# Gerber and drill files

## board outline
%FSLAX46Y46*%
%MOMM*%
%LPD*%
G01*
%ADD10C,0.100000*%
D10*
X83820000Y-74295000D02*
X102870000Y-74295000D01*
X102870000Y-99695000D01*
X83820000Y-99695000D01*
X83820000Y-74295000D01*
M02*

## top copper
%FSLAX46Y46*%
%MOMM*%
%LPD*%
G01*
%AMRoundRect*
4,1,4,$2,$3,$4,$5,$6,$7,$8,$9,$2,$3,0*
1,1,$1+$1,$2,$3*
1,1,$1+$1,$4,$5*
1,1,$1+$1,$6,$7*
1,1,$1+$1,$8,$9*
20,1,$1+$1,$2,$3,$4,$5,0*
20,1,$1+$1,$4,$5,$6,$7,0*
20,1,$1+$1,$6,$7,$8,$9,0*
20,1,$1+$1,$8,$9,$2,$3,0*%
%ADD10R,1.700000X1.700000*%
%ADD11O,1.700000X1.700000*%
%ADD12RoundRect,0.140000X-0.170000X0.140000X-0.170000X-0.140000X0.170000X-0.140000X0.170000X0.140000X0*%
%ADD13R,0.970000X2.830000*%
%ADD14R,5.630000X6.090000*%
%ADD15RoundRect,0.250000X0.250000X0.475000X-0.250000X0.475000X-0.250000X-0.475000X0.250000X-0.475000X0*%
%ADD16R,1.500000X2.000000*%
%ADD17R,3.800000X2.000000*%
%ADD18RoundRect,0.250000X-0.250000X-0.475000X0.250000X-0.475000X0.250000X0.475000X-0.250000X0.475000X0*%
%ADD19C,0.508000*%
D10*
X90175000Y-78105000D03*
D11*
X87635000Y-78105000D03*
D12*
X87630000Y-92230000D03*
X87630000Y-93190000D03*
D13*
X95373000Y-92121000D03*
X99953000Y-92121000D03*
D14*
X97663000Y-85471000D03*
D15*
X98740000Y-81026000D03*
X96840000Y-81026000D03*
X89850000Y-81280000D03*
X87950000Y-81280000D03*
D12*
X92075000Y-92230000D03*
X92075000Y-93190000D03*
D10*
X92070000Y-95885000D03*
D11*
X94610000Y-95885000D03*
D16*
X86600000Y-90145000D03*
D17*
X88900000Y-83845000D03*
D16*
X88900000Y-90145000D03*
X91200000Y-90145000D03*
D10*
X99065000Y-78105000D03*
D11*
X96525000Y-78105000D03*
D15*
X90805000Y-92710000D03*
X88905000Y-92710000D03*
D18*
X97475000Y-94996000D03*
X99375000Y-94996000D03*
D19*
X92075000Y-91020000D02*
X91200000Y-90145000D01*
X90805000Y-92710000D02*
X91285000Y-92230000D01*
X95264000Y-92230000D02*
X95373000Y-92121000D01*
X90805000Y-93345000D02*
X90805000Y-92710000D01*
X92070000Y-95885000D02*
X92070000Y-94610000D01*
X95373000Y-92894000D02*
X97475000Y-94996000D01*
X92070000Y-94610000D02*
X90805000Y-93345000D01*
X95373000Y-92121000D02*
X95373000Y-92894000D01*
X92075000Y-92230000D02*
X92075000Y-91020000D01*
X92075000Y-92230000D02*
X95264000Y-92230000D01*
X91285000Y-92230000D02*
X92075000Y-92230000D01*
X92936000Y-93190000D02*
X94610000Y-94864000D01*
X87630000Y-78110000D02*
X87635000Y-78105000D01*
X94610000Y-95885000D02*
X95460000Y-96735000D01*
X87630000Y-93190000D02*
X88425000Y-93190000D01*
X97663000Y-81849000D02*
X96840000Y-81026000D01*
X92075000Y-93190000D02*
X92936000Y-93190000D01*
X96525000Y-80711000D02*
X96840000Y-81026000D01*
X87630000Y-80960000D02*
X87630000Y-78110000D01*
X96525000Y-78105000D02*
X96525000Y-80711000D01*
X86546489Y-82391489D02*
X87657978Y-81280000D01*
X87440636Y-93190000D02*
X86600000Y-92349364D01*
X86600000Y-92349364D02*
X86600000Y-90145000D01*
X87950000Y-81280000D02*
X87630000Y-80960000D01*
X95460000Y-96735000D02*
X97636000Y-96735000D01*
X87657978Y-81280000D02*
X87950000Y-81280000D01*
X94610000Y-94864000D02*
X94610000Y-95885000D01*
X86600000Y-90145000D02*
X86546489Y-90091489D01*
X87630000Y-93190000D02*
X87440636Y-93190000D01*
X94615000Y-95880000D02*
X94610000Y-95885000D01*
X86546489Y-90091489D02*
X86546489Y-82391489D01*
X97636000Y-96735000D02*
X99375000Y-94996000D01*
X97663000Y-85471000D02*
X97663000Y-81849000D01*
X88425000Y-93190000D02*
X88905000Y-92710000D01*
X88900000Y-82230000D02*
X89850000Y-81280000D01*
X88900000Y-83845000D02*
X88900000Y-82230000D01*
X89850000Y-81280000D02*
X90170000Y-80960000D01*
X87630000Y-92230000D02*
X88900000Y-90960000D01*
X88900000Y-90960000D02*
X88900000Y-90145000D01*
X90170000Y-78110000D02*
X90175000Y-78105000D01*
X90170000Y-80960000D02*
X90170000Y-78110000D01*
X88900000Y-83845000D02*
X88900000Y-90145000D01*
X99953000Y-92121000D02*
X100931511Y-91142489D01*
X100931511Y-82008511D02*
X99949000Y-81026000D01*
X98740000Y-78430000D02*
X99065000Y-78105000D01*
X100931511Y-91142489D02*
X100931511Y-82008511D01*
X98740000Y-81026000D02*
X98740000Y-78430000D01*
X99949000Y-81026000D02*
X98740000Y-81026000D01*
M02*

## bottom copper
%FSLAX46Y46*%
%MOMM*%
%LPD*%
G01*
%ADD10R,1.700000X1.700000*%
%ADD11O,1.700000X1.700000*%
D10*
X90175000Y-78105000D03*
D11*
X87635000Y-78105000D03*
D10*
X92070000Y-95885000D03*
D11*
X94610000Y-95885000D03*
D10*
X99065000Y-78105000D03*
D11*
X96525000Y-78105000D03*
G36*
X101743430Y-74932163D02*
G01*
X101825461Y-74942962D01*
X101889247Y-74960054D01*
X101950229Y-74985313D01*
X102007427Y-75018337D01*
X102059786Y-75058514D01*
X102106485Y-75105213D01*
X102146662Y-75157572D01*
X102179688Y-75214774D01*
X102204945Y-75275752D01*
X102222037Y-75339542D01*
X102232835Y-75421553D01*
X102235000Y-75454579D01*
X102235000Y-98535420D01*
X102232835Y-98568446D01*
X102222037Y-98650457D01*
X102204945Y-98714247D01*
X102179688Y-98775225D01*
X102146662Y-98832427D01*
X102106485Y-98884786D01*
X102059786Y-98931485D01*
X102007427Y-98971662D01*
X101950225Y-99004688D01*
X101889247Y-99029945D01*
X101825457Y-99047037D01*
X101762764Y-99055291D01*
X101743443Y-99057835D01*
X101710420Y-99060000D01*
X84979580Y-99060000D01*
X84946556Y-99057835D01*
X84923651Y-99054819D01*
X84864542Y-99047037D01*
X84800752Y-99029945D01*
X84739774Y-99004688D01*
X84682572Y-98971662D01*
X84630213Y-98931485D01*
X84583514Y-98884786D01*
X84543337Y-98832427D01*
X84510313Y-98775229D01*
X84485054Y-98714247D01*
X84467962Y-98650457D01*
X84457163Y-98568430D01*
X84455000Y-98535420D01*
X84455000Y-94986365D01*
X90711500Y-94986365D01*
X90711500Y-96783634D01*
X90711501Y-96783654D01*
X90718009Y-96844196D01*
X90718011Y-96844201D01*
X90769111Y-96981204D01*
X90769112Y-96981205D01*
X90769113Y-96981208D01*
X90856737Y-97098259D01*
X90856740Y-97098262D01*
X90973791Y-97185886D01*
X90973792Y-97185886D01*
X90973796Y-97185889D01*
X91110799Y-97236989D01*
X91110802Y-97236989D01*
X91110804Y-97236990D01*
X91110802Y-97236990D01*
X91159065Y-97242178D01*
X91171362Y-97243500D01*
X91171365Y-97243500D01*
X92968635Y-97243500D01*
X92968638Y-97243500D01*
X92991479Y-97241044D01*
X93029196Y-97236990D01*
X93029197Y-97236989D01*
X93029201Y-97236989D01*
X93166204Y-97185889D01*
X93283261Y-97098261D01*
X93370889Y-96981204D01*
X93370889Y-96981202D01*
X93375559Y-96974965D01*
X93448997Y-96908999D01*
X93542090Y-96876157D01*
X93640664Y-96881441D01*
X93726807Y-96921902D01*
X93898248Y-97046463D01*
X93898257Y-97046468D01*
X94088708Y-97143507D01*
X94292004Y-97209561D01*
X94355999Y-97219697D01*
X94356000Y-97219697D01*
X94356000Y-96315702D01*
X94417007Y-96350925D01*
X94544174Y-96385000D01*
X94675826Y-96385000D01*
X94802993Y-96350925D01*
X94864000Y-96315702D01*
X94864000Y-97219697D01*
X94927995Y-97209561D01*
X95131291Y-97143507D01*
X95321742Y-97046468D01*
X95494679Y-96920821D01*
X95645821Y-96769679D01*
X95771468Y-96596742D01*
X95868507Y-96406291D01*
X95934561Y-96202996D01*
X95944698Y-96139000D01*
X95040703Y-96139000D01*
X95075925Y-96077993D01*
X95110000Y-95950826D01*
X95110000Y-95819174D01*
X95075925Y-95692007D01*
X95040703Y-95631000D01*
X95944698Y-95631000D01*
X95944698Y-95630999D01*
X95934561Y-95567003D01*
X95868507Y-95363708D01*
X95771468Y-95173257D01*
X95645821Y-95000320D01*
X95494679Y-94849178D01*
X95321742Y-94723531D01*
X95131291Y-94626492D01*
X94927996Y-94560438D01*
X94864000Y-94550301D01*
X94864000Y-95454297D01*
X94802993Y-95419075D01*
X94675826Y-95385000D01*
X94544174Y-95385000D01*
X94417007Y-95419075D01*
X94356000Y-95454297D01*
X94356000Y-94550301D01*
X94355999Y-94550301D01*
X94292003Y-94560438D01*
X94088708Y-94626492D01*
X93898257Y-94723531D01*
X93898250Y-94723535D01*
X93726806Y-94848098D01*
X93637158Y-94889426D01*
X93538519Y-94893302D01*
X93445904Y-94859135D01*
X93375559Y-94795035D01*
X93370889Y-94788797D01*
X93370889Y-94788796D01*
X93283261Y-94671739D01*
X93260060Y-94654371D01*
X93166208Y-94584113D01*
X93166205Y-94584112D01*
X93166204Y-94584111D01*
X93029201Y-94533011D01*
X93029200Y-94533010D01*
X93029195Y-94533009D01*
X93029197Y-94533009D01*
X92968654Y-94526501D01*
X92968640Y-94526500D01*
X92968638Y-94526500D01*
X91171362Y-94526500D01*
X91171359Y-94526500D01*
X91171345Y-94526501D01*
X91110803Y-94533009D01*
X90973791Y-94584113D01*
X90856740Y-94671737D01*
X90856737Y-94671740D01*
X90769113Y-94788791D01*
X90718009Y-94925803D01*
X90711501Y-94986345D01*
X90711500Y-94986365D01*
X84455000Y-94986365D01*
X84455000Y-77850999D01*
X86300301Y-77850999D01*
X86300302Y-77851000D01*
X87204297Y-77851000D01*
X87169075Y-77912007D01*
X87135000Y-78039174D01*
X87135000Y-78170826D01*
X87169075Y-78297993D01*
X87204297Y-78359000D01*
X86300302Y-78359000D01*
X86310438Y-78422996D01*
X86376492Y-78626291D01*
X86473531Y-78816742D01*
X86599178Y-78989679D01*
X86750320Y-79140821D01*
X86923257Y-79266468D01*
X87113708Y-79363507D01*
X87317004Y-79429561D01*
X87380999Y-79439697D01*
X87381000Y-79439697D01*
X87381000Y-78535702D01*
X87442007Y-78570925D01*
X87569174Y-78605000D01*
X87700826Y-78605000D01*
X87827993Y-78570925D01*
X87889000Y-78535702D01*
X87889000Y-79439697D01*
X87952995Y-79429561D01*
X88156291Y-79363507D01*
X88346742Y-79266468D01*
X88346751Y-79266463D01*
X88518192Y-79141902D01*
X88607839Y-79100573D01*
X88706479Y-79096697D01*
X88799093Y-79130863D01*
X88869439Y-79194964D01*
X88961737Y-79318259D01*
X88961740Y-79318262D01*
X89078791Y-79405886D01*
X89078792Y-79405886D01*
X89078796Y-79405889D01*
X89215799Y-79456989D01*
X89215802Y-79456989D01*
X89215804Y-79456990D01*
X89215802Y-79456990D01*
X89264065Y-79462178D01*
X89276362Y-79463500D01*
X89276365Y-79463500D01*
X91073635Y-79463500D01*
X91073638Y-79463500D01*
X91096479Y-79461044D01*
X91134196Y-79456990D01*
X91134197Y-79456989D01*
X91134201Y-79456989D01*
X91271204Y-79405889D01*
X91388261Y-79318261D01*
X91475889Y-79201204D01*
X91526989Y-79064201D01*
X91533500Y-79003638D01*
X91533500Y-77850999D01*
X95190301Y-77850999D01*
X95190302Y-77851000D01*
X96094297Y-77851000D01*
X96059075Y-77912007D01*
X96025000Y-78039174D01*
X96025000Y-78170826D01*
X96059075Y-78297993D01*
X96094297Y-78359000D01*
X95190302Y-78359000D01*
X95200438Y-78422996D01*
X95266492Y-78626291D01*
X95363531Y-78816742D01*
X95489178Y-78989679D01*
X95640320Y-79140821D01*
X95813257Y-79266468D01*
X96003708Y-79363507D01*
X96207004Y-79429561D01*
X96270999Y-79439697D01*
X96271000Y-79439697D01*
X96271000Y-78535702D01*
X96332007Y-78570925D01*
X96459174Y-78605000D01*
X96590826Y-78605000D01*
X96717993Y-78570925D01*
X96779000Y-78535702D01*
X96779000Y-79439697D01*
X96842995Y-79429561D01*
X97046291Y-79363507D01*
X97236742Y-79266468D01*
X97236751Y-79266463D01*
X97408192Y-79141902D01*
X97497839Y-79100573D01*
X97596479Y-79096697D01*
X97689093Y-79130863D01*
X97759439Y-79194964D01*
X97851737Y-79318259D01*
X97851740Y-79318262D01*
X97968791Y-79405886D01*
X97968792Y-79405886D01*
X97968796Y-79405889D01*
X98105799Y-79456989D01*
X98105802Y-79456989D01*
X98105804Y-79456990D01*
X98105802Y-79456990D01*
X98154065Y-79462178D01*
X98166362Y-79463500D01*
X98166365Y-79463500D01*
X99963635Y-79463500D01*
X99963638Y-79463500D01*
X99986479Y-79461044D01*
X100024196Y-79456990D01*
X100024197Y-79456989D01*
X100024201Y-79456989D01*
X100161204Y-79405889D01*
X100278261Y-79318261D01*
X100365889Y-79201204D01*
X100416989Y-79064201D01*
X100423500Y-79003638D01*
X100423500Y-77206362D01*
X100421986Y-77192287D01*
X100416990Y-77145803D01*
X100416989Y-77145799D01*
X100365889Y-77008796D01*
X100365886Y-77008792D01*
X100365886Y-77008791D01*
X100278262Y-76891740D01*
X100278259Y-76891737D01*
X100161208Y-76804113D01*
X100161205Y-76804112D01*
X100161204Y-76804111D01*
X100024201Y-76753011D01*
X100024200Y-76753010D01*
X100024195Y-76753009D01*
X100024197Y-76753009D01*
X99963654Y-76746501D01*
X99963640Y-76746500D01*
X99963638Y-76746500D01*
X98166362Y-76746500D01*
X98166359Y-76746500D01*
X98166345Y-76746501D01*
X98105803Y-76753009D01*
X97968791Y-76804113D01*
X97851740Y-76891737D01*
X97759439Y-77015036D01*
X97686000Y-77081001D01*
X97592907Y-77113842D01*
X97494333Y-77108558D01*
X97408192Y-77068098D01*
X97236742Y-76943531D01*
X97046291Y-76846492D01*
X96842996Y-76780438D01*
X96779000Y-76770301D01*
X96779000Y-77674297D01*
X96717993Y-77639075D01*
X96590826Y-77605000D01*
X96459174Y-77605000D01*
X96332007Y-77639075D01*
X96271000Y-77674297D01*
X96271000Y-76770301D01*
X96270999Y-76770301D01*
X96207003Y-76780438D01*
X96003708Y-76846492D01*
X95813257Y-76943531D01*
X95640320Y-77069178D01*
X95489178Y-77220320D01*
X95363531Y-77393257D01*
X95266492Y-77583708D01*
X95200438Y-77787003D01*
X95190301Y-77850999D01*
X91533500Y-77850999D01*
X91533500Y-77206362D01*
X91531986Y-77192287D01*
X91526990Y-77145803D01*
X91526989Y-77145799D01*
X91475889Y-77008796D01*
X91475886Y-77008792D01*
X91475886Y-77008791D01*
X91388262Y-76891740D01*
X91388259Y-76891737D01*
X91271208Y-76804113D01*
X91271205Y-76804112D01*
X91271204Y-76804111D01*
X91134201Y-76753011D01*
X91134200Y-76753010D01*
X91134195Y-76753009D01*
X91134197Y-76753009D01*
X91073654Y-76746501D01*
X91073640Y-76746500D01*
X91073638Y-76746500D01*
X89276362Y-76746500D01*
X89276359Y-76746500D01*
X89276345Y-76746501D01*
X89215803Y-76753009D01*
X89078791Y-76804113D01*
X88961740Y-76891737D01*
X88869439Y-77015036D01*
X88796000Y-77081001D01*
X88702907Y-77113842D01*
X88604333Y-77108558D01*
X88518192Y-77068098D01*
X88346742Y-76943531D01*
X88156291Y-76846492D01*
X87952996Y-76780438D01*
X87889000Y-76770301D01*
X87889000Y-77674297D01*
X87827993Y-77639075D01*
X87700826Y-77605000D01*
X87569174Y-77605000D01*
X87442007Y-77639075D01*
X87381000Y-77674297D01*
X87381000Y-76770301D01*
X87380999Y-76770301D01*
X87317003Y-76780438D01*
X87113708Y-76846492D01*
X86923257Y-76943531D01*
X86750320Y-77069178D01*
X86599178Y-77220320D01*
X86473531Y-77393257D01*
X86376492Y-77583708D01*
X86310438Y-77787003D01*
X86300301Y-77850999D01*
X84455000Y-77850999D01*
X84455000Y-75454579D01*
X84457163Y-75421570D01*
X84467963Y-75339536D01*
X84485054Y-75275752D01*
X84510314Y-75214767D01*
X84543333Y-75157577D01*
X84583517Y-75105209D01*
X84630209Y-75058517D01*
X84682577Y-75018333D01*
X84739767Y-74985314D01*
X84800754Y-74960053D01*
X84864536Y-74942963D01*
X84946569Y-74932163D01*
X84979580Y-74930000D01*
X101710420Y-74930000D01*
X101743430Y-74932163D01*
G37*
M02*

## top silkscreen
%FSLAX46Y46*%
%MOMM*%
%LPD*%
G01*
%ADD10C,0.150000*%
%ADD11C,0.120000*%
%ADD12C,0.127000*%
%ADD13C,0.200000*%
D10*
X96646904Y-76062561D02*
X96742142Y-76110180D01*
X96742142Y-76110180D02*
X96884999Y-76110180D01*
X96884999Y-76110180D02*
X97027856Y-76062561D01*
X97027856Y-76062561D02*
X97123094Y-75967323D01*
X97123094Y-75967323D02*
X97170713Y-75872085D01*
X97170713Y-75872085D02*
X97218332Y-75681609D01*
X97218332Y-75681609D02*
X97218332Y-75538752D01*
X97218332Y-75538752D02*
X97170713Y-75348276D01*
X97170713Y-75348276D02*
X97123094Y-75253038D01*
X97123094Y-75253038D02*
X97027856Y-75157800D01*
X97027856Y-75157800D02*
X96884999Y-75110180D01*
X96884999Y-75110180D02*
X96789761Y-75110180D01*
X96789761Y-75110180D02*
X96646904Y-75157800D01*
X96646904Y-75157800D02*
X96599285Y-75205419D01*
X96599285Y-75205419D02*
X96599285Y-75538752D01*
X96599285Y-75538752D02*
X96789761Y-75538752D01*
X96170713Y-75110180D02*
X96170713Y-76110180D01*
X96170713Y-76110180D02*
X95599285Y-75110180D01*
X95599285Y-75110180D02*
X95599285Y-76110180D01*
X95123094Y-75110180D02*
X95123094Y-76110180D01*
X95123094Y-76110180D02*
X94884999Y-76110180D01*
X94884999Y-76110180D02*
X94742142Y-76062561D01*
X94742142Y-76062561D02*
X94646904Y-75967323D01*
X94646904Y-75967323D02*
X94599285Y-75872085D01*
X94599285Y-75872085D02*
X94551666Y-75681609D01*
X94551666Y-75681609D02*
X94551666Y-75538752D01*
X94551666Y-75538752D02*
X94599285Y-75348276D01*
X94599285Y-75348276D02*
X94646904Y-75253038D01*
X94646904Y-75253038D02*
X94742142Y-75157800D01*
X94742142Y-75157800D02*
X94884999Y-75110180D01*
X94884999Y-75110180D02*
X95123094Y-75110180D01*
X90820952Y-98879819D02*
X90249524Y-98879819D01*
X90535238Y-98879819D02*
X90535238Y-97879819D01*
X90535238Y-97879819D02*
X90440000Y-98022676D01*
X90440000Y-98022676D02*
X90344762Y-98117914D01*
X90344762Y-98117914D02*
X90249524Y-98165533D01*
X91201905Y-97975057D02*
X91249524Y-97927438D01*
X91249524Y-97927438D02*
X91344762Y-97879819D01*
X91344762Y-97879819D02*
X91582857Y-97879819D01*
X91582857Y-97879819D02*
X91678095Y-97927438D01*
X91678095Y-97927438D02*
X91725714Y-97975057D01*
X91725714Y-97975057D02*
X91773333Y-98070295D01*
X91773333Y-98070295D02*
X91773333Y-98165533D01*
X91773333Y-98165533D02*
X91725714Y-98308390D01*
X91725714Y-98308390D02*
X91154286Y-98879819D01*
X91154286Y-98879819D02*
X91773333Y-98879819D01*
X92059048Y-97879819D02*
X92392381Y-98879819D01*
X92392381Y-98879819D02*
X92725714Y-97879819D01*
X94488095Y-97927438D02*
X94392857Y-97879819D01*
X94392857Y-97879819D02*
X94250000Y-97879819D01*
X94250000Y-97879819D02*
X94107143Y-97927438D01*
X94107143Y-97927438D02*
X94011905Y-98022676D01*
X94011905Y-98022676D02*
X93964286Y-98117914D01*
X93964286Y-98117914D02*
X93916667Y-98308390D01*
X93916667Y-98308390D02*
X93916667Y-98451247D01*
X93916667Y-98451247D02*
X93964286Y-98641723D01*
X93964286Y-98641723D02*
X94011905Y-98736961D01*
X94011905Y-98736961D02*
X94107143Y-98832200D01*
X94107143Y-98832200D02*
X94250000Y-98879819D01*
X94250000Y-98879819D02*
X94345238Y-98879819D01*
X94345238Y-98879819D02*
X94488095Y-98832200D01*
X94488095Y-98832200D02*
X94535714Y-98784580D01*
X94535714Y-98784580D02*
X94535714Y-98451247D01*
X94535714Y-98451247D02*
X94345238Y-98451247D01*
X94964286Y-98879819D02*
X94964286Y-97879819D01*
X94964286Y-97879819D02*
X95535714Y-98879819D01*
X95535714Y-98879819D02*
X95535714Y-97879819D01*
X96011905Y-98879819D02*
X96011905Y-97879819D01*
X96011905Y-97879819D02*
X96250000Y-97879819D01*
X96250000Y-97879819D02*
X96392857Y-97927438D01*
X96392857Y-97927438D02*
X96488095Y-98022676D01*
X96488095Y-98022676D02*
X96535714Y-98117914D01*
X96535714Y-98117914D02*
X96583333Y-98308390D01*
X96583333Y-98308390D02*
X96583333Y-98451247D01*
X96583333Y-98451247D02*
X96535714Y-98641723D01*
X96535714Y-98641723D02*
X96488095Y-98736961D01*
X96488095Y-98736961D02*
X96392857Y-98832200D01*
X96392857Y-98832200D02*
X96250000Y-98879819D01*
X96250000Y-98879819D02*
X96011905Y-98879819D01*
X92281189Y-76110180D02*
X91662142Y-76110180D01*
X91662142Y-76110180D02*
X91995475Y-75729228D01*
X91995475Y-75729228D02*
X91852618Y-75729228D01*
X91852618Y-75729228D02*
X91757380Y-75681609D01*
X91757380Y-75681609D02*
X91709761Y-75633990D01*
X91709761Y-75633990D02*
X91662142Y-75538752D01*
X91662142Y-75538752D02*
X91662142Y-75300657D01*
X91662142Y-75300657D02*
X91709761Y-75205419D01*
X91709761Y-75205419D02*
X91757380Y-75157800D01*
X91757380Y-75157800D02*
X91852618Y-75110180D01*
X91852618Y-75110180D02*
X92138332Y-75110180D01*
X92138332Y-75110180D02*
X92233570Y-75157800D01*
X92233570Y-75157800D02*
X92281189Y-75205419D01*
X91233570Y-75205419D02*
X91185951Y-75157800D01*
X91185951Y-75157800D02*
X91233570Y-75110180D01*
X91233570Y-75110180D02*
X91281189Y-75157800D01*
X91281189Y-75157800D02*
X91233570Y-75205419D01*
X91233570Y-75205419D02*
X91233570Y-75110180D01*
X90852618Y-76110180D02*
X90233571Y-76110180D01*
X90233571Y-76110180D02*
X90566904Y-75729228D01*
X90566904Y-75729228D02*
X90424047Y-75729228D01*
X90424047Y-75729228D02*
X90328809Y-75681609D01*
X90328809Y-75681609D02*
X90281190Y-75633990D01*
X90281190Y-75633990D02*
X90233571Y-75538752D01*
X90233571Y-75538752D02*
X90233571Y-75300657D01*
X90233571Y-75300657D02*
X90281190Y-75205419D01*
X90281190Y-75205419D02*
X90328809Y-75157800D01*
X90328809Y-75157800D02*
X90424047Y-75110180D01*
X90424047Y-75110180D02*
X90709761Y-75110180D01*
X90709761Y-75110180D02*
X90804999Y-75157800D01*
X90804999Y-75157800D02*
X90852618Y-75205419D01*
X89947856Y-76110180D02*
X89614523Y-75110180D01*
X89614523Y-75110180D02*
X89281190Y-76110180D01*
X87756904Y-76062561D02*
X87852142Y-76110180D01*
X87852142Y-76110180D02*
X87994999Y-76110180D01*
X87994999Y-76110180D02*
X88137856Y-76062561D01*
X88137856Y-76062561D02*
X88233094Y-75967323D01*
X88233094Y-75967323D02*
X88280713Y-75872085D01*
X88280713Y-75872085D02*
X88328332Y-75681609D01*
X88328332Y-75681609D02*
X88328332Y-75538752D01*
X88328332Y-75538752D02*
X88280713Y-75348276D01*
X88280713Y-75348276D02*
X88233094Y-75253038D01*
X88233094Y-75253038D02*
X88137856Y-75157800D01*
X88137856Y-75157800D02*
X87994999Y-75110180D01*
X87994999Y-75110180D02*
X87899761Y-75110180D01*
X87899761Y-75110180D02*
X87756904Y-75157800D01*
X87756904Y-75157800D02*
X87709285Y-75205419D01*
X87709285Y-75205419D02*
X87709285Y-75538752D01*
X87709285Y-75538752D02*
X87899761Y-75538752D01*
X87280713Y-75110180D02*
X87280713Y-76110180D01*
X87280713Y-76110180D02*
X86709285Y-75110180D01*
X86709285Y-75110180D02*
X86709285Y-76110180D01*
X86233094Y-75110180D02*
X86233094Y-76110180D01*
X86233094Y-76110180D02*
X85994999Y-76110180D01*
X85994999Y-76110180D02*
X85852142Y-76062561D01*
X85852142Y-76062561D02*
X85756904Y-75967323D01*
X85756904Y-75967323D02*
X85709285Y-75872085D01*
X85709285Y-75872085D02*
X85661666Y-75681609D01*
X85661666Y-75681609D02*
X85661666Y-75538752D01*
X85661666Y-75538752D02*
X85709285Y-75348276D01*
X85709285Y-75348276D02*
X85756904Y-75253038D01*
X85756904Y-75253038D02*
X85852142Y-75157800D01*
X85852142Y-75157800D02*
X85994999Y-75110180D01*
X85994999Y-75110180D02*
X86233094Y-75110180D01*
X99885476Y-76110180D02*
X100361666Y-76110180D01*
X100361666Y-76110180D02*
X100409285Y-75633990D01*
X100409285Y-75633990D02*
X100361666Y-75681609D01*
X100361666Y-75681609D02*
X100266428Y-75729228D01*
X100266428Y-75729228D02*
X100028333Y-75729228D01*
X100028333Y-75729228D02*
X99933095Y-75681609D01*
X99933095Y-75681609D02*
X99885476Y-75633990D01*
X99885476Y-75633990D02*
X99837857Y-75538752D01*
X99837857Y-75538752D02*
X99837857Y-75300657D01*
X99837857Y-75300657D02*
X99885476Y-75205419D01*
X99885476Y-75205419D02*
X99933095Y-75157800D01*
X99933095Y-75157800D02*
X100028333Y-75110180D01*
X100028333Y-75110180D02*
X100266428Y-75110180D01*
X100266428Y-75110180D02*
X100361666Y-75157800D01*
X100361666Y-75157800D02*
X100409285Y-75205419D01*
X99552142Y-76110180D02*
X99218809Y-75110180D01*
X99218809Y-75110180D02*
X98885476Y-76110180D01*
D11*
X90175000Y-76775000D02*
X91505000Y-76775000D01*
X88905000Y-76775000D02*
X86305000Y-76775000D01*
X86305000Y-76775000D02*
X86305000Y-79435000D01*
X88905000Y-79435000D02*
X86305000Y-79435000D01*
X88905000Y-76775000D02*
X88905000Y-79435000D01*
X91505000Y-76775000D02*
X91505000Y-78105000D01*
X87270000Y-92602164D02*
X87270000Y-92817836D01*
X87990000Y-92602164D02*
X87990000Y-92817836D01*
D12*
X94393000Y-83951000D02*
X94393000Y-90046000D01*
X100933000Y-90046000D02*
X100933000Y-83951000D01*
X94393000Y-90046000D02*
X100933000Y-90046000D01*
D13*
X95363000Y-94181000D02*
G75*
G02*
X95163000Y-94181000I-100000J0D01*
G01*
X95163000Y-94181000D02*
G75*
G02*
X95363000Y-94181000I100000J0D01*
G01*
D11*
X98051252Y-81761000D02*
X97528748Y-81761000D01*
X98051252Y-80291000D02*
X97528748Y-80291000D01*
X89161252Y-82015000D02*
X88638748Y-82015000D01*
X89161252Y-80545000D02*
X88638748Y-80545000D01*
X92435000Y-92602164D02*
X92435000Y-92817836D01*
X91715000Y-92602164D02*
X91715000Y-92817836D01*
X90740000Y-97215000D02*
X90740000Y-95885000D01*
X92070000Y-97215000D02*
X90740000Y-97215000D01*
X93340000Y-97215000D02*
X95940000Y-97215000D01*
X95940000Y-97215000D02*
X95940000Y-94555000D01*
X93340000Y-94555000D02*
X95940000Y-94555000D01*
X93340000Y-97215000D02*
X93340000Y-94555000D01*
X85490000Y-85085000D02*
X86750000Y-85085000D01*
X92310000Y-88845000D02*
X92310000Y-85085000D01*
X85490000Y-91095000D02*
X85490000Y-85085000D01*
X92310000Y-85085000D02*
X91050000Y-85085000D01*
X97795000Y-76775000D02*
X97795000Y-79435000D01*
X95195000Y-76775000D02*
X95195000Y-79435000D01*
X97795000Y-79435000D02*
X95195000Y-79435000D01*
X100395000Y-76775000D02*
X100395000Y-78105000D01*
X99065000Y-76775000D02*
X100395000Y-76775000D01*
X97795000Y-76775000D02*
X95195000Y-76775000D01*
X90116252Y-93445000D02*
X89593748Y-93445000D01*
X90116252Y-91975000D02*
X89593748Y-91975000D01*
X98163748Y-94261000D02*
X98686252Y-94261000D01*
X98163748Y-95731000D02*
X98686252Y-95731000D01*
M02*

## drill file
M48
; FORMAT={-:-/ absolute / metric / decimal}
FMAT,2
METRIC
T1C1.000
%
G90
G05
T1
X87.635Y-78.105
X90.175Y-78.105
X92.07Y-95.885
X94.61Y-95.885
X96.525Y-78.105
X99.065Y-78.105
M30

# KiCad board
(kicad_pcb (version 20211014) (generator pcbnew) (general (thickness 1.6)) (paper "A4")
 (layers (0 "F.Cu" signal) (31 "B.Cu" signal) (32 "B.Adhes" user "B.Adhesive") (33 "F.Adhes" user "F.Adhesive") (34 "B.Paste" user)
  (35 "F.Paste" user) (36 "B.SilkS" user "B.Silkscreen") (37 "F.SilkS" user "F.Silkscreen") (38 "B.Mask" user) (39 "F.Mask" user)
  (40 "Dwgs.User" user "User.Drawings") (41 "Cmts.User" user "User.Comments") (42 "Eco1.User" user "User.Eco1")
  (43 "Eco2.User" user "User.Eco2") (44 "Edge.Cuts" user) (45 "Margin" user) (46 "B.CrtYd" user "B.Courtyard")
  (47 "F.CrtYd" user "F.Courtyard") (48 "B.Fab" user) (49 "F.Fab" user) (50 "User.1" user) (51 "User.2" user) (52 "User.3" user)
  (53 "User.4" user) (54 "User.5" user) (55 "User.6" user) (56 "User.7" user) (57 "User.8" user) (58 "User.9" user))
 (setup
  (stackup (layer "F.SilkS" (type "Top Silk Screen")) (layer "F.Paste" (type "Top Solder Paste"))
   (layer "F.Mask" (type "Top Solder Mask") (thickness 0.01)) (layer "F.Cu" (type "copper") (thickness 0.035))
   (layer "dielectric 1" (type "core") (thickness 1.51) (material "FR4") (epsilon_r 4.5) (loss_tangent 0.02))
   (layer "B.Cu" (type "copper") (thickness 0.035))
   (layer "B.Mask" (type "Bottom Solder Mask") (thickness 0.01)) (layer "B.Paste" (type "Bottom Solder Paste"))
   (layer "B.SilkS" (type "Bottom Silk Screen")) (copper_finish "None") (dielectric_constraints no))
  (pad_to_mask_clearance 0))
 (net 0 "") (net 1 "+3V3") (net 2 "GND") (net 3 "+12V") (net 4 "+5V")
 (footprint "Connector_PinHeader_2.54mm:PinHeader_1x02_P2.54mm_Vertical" (layer "F.Cu") (at 90.175 78.105 -90)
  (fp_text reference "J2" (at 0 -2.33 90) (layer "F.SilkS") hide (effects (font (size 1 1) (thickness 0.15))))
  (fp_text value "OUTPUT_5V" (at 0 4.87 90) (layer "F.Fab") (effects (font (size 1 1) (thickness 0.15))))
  (fp_line (start -1.33 0) (end -1.33 -1.33) (layer "F.SilkS") (width 0.12))
  (fp_line (start -1.33 1.27) (end -1.33 3.87) (layer "F.SilkS") (width 0.12))
  (fp_line (start -1.33 3.87) (end 1.33 3.87) (layer "F.SilkS") (width 0.12))
  (fp_line (start 1.33 1.27) (end 1.33 3.87) (layer "F.SilkS") (width 0.12))
  (fp_line (start -1.33 1.27) (end 1.33 1.27) (layer "F.SilkS") (width 0.12))
  (fp_line (start -1.33 -1.33) (end 0 -1.33) (layer "F.SilkS") (width 0.12))
  (pad "1" thru_hole rect (at 0 0 270) (size 1.7 1.7) (drill 1) (layers *.Cu *.Mask) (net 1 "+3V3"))
  (pad "2" thru_hole oval (at 0 2.54 270) (size 1.7 1.7) (drill 1) (layers *.Cu *.Mask) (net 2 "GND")))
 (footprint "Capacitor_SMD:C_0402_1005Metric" (layer "F.Cu") (at 87.63 92.71 -90)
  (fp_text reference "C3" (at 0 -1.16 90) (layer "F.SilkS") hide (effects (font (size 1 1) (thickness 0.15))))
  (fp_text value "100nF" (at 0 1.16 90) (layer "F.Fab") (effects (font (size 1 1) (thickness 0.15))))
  (fp_line (start -0.107836 0.36) (end 0.107836 0.36) (layer "F.SilkS") (width 0.12))
  (fp_line (start -0.107836 -0.36) (end 0.107836 -0.36) (layer "F.SilkS") (width 0.12))
  (pad "1" smd roundrect (at -0.48 0 270) (size 0.56 0.62) (layers "F.Cu" "F.Paste" "F.Mask") (roundrect_rratio 0.25) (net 1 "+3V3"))
  (pad "2" smd roundrect (at 0.48 0 270) (size 0.56 0.62) (layers "F.Cu" "F.Paste" "F.Mask") (roundrect_rratio 0.25) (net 2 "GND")))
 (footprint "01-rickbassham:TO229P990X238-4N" (layer "F.Cu") (at 97.663 87.981 90)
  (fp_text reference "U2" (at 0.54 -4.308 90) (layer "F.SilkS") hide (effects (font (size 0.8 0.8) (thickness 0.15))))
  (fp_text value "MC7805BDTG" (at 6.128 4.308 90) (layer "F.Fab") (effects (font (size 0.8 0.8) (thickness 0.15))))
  (fp_line (start 4.03 -3.27) (end -2.065 -3.27) (layer "F.SilkS") (width 0.127))
  (fp_line (start -2.065 3.27) (end 4.03 3.27) (layer "F.SilkS") (width 0.127))
  (fp_line (start -2.065 -3.27) (end -2.065 3.27) (layer "F.SilkS") (width 0.127))
  (fp_circle (center -6.2 -2.4) (end -6.1 -2.4) (layer "F.SilkS") (width 0.2) (fill none))
  (pad "1" smd rect (at -4.14 -2.29 90) (size 2.83 0.97) (layers "F.Cu" "F.Paste" "F.Mask") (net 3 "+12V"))
  (pad "3" smd rect (at -4.14 2.29 90) (size 2.83 0.97) (layers "F.Cu" "F.Paste" "F.Mask") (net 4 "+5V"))
  (pad "4" smd rect (at 2.51 0 90) (size 6.09 5.63) (layers "F.Cu" "F.Mask") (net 2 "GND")))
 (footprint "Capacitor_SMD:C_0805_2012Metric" (layer "F.Cu") (at 97.79 81.026 180)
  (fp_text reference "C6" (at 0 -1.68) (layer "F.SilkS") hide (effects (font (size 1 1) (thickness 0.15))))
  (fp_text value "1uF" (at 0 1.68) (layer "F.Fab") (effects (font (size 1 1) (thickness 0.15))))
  (fp_line (start -0.261252 -0.735) (end 0.261252 -0.735) (layer "F.SilkS") (width 0.12))
  (fp_line (start -0.261252 0.735) (end 0.261252 0.735) (layer "F.SilkS") (width 0.12))
  (pad "1" smd roundrect (at -0.95 0 180) (size 1 1.45) (layers "F.Cu" "F.Paste" "F.Mask") (roundrect_rratio 0.25) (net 4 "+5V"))
  (pad "2" smd roundrect (at 0.95 0 180) (size 1 1.45) (layers "F.Cu" "F.Paste" "F.Mask") (roundrect_rratio 0.25) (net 2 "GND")))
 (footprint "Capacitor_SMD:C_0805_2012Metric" (layer "F.Cu") (at 88.9 81.28 180)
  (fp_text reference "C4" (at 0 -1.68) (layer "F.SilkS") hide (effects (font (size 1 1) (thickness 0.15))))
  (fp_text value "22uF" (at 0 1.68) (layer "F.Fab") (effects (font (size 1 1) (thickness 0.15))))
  (fp_line (start -0.261252 -0.735) (end 0.261252 -0.735) (layer "F.SilkS") (width 0.12))
  (fp_line (start -0.261252 0.735) (end 0.261252 0.735) (layer "F.SilkS") (width 0.12))
  (pad "1" smd roundrect (at -0.95 0 180) (size 1 1.45) (layers "F.Cu" "F.Paste" "F.Mask") (roundrect_rratio 0.25) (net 1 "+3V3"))
  (pad "2" smd roundrect (at 0.95 0 180) (size 1 1.45) (layers "F.Cu" "F.Paste" "F.Mask") (roundrect_rratio 0.25) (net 2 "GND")))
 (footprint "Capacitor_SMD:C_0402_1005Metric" (layer "F.Cu") (at 92.075 92.71 -90)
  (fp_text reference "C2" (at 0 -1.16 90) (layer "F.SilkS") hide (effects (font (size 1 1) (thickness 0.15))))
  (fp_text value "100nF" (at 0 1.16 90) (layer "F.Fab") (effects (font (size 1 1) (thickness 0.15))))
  (fp_line (start -0.107836 -0.36) (end 0.107836 -0.36) (layer "F.SilkS") (width 0.12))
  (fp_line (start -0.107836 0.36) (end 0.107836 0.36) (layer "F.SilkS") (width 0.12))
  (pad "1" smd roundrect (at -0.48 0 270) (size 0.56 0.62) (layers "F.Cu" "F.Paste" "F.Mask") (roundrect_rratio 0.25) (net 3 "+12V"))
  (pad "2" smd roundrect (at 0.48 0 270) (size 0.56 0.62) (layers "F.Cu" "F.Paste" "F.Mask") (roundrect_rratio 0.25) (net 2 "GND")))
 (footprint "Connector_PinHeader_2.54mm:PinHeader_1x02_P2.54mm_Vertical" (layer "F.Cu") (at 92.07 95.885 90)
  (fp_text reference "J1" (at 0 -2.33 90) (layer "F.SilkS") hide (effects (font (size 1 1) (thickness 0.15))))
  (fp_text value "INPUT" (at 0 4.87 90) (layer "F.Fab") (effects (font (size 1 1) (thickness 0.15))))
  (fp_line (start -1.33 -1.33) (end 0 -1.33) (layer "F.SilkS") (width 0.12))
  (fp_line (start -1.33 0) (end -1.33 -1.33) (layer "F.SilkS") (width 0.12))
  (fp_line (start -1.33 1.27) (end -1.33 3.87) (layer "F.SilkS") (width 0.12))
  (fp_line (start -1.33 3.87) (end 1.33 3.87) (layer "F.SilkS") (width 0.12))
  (fp_line (start 1.33 1.27) (end 1.33 3.87) (layer "F.SilkS") (width 0.12))
  (fp_line (start -1.33 1.27) (end 1.33 1.27) (layer "F.SilkS") (width 0.12))
  (pad "1" thru_hole rect (at 0 0 90) (size 1.7 1.7) (drill 1) (layers *.Cu *.Mask) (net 3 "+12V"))
  (pad "2" thru_hole oval (at 0 2.54 90) (size 1.7 1.7) (drill 1) (layers *.Cu *.Mask) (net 2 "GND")))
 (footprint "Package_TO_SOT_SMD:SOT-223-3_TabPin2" (layer "F.Cu") (at 88.9 86.995 90)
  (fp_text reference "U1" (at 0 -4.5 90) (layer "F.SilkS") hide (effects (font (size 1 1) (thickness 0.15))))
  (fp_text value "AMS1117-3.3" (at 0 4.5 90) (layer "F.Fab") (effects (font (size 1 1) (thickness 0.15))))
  (fp_line (start 1.91 -3.41) (end 1.91 -2.15) (layer "F.SilkS") (width 0.12))
  (fp_line (start -1.85 3.41) (end 1.91 3.41) (layer "F.SilkS") (width 0.12))
  (fp_line (start -4.1 -3.41) (end 1.91 -3.41) (layer "F.SilkS") (width 0.12))
  (fp_line (start 1.91 3.41) (end 1.91 2.15) (layer "F.SilkS") (width 0.12))
  (pad "1" smd rect (at -3.15 -2.3 90) (size 2 1.5) (layers "F.Cu" "F.Paste" "F.Mask") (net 2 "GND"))
  (pad "2" smd rect (at 3.15 0 90) (size 2 3.8) (layers "F.Cu" "F.Paste" "F.Mask") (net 1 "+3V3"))
  (pad "2" smd rect (at -3.15 0 90) (size 2 1.5) (layers "F.Cu" "F.Paste" "F.Mask") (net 1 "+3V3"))
  (pad "3" smd rect (at -3.15 2.3 90) (size 2 1.5) (layers "F.Cu" "F.Paste" "F.Mask") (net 3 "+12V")))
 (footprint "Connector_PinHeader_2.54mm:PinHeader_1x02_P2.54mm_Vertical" (layer "F.Cu") (at 99.065 78.105 -90)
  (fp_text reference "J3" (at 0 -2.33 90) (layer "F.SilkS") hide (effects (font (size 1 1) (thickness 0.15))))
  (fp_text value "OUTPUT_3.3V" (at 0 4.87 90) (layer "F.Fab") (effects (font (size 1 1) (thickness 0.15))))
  (fp_line (start -1.33 1.27) (end 1.33 1.27) (layer "F.SilkS") (width 0.12))
  (fp_line (start -1.33 3.87) (end 1.33 3.87) (layer "F.SilkS") (width 0.12))
  (fp_line (start 1.33 1.27) (end 1.33 3.87) (layer "F.SilkS") (width 0.12))
  (fp_line (start -1.33 -1.33) (end 0 -1.33) (layer "F.SilkS") (width 0.12))
  (fp_line (start -1.33 0) (end -1.33 -1.33) (layer "F.SilkS") (width 0.12))
  (fp_line (start -1.33 1.27) (end -1.33 3.87) (layer "F.SilkS") (width 0.12))
  (pad "1" thru_hole rect (at 0 0 270) (size 1.7 1.7) (drill 1) (layers *.Cu *.Mask) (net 4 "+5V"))
  (pad "2" thru_hole oval (at 0 2.54 270) (size 1.7 1.7) (drill 1) (layers *.Cu *.Mask) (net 2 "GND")))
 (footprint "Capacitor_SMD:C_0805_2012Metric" (layer "F.Cu") (at 89.855 92.71 180)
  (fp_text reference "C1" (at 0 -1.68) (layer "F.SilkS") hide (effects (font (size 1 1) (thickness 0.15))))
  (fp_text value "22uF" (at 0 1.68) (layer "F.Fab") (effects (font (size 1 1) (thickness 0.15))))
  (fp_line (start -0.261252 -0.735) (end 0.261252 -0.735) (layer "F.SilkS") (width 0.12))
  (fp_line (start -0.261252 0.735) (end 0.261252 0.735) (layer "F.SilkS") (width 0.12))
  (pad "1" smd roundrect (at -0.95 0 180) (size 1 1.45) (layers "F.Cu" "F.Paste" "F.Mask") (roundrect_rratio 0.25) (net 3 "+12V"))
  (pad "2" smd roundrect (at 0.95 0 180) (size 1 1.45) (layers "F.Cu" "F.Paste" "F.Mask") (roundrect_rratio 0.25) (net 2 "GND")))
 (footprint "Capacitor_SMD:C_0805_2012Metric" (layer "F.Cu") (at 98.425 94.996)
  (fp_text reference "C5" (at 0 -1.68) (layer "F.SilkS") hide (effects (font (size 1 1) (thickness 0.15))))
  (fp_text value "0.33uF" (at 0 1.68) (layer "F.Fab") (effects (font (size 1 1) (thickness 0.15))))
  (fp_line (start -0.261252 -0.735) (end 0.261252 -0.735) (layer "F.SilkS") (width 0.12))
  (fp_line (start -0.261252 0.735) (end 0.261252 0.735) (layer "F.SilkS") (width 0.12))
  (pad "1" smd roundrect (at -0.95 0) (size 1 1.45) (layers "F.Cu" "F.Paste" "F.Mask") (roundrect_rratio 0.25) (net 3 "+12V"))
  (pad "2" smd roundrect (at 0.95 0) (size 1 1.45) (layers "F.Cu" "F.Paste" "F.Mask") (roundrect_rratio 0.25) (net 2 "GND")))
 (gr_rect (start 83.82 74.295) (end 102.87 99.695) (layer "Edge.Cuts") (width 0.1) (fill none))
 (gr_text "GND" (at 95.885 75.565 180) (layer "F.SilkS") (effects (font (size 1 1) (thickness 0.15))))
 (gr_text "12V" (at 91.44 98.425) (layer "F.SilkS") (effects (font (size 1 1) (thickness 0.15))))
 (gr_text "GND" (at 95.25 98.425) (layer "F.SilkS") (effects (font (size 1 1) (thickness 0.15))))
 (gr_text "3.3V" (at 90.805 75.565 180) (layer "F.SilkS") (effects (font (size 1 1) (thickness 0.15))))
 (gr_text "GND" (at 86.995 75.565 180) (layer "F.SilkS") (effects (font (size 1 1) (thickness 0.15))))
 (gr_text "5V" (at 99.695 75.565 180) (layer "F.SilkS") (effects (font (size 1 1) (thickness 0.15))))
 (segment (start 92.075 91.02) (end 91.2 90.145) (width 0.508) (layer "F.Cu") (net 3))
 (segment (start 90.805 92.71) (end 91.285 92.23) (width 0.508) (layer "F.Cu") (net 3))
 (segment (start 95.264 92.23) (end 95.373 92.121) (width 0.508) (layer "F.Cu") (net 3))
 (segment (start 90.805 93.345) (end 90.805 92.71) (width 0.508) (layer "F.Cu") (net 3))
 (segment (start 92.07 95.885) (end 92.07 94.61) (width 0.508) (layer "F.Cu") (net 3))
 (segment (start 95.373 92.894) (end 97.475 94.996) (width 0.508) (layer "F.Cu") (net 3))
 (segment (start 92.07 94.61) (end 90.805 93.345) (width 0.508) (layer "F.Cu") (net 3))
 (segment (start 95.373 92.121) (end 95.373 92.894) (width 0.508) (layer "F.Cu") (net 3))
 (segment (start 92.075 92.23) (end 92.075 91.02) (width 0.508) (layer "F.Cu") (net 3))
 (segment (start 92.075 92.23) (end 95.264 92.23) (width 0.508) (layer "F.Cu") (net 3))
 (segment (start 91.285 92.23) (end 92.075 92.23) (width 0.508) (layer "F.Cu") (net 3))
 (segment (start 92.936 93.19) (end 94.61 94.864) (width 0.508) (layer "F.Cu") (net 2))
 (segment (start 87.63 78.11) (end 87.635 78.105) (width 0.508) (layer "F.Cu") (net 2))
 (segment (start 94.61 95.885) (end 95.46 96.735) (width 0.508) (layer "F.Cu") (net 2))
 (segment (start 87.63 93.19) (end 88.425 93.19) (width 0.508) (layer "F.Cu") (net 2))
 (segment (start 97.663 81.849) (end 96.84 81.026) (width 0.508) (layer "F.Cu") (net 2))
 (segment (start 92.075 93.19) (end 92.936 93.19) (width 0.508) (layer "F.Cu") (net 2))
 (segment (start 96.525 80.711) (end 96.84 81.026) (width 0.508) (layer "F.Cu") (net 2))
 (segment (start 87.63 80.96) (end 87.63 78.11) (width 0.508) (layer "F.Cu") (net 2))
 (segment (start 96.525 78.105) (end 96.525 80.711) (width 0.508) (layer "F.Cu") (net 2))
 (segment (start 86.546489 82.391489) (end 87.657978 81.28) (width 0.508) (layer "F.Cu") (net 2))
 (segment (start 87.440636 93.19) (end 86.6 92.349364) (width 0.508) (layer "F.Cu") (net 2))
 (segment (start 86.6 92.349364) (end 86.6 90.145) (width 0.508) (layer "F.Cu") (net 2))
 (segment (start 87.95 81.28) (end 87.63 80.96) (width 0.508) (layer "F.Cu") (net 2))
 (segment (start 95.46 96.735) (end 97.636 96.735) (width 0.508) (layer "F.Cu") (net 2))
 (segment (start 87.657978 81.28) (end 87.95 81.28) (width 0.508) (layer "F.Cu") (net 2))
 (segment (start 94.61 94.864) (end 94.61 95.885) (width 0.508) (layer "F.Cu") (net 2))
 (segment (start 86.6 90.145) (end 86.546489 90.091489) (width 0.508) (layer "F.Cu") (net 2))
 (segment (start 87.63 93.19) (end 87.440636 93.19) (width 0.508) (layer "F.Cu") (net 2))
 (segment (start 94.615 95.88) (end 94.61 95.885) (width 0.508) (layer "F.Cu") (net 2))
 (segment (start 86.546489 90.091489) (end 86.546489 82.391489) (width 0.508) (layer "F.Cu") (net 2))
 (segment (start 97.636 96.735) (end 99.375 94.996) (width 0.508) (layer "F.Cu") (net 2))
 (segment (start 97.663 85.471) (end 97.663 81.849) (width 0.508) (layer "F.Cu") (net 2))
 (segment (start 88.425 93.19) (end 88.905 92.71) (width 0.508) (layer "F.Cu") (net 2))
 (segment (start 88.9 82.23) (end 89.85 81.28) (width 0.508) (layer "F.Cu") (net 1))
 (segment (start 88.9 83.845) (end 88.9 82.23) (width 0.508) (layer "F.Cu") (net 1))
 (segment (start 89.85 81.28) (end 90.17 80.96) (width 0.508) (layer "F.Cu") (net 1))
 (segment (start 87.63 92.23) (end 88.9 90.96) (width 0.508) (layer "F.Cu") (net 1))
 (segment (start 88.9 90.96) (end 88.9 90.145) (width 0.508) (layer "F.Cu") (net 1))
 (segment (start 90.17 78.11) (end 90.175 78.105) (width 0.508) (layer "F.Cu") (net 1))
 (segment (start 90.17 80.96) (end 90.17 78.11) (width 0.508) (layer "F.Cu") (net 1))
 (segment (start 88.9 83.845) (end 88.9 90.145) (width 0.508) (layer "F.Cu") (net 1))
 (segment (start 99.953 92.121) (end 100.931511 91.142489) (width 0.508) (layer "F.Cu") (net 4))
 (segment (start 100.931511 82.008511) (end 99.949 81.026) (width 0.508) (layer "F.Cu") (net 4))
 (segment (start 98.74 78.43) (end 99.065 78.105) (width 0.508) (layer "F.Cu") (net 4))
 (segment (start 100.931511 91.142489) (end 100.931511 82.008511) (width 0.508) (layer "F.Cu") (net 4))
 (segment (start 98.74 81.026) (end 98.74 78.43) (width 0.508) (layer "F.Cu") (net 4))
 (segment (start 99.949 81.026) (end 98.74 81.026) (width 0.508) (layer "F.Cu") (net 4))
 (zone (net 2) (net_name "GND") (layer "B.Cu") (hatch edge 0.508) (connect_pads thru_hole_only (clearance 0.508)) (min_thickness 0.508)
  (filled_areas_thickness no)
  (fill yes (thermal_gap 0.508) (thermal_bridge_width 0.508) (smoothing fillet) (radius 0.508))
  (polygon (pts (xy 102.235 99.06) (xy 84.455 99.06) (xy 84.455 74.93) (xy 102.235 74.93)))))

